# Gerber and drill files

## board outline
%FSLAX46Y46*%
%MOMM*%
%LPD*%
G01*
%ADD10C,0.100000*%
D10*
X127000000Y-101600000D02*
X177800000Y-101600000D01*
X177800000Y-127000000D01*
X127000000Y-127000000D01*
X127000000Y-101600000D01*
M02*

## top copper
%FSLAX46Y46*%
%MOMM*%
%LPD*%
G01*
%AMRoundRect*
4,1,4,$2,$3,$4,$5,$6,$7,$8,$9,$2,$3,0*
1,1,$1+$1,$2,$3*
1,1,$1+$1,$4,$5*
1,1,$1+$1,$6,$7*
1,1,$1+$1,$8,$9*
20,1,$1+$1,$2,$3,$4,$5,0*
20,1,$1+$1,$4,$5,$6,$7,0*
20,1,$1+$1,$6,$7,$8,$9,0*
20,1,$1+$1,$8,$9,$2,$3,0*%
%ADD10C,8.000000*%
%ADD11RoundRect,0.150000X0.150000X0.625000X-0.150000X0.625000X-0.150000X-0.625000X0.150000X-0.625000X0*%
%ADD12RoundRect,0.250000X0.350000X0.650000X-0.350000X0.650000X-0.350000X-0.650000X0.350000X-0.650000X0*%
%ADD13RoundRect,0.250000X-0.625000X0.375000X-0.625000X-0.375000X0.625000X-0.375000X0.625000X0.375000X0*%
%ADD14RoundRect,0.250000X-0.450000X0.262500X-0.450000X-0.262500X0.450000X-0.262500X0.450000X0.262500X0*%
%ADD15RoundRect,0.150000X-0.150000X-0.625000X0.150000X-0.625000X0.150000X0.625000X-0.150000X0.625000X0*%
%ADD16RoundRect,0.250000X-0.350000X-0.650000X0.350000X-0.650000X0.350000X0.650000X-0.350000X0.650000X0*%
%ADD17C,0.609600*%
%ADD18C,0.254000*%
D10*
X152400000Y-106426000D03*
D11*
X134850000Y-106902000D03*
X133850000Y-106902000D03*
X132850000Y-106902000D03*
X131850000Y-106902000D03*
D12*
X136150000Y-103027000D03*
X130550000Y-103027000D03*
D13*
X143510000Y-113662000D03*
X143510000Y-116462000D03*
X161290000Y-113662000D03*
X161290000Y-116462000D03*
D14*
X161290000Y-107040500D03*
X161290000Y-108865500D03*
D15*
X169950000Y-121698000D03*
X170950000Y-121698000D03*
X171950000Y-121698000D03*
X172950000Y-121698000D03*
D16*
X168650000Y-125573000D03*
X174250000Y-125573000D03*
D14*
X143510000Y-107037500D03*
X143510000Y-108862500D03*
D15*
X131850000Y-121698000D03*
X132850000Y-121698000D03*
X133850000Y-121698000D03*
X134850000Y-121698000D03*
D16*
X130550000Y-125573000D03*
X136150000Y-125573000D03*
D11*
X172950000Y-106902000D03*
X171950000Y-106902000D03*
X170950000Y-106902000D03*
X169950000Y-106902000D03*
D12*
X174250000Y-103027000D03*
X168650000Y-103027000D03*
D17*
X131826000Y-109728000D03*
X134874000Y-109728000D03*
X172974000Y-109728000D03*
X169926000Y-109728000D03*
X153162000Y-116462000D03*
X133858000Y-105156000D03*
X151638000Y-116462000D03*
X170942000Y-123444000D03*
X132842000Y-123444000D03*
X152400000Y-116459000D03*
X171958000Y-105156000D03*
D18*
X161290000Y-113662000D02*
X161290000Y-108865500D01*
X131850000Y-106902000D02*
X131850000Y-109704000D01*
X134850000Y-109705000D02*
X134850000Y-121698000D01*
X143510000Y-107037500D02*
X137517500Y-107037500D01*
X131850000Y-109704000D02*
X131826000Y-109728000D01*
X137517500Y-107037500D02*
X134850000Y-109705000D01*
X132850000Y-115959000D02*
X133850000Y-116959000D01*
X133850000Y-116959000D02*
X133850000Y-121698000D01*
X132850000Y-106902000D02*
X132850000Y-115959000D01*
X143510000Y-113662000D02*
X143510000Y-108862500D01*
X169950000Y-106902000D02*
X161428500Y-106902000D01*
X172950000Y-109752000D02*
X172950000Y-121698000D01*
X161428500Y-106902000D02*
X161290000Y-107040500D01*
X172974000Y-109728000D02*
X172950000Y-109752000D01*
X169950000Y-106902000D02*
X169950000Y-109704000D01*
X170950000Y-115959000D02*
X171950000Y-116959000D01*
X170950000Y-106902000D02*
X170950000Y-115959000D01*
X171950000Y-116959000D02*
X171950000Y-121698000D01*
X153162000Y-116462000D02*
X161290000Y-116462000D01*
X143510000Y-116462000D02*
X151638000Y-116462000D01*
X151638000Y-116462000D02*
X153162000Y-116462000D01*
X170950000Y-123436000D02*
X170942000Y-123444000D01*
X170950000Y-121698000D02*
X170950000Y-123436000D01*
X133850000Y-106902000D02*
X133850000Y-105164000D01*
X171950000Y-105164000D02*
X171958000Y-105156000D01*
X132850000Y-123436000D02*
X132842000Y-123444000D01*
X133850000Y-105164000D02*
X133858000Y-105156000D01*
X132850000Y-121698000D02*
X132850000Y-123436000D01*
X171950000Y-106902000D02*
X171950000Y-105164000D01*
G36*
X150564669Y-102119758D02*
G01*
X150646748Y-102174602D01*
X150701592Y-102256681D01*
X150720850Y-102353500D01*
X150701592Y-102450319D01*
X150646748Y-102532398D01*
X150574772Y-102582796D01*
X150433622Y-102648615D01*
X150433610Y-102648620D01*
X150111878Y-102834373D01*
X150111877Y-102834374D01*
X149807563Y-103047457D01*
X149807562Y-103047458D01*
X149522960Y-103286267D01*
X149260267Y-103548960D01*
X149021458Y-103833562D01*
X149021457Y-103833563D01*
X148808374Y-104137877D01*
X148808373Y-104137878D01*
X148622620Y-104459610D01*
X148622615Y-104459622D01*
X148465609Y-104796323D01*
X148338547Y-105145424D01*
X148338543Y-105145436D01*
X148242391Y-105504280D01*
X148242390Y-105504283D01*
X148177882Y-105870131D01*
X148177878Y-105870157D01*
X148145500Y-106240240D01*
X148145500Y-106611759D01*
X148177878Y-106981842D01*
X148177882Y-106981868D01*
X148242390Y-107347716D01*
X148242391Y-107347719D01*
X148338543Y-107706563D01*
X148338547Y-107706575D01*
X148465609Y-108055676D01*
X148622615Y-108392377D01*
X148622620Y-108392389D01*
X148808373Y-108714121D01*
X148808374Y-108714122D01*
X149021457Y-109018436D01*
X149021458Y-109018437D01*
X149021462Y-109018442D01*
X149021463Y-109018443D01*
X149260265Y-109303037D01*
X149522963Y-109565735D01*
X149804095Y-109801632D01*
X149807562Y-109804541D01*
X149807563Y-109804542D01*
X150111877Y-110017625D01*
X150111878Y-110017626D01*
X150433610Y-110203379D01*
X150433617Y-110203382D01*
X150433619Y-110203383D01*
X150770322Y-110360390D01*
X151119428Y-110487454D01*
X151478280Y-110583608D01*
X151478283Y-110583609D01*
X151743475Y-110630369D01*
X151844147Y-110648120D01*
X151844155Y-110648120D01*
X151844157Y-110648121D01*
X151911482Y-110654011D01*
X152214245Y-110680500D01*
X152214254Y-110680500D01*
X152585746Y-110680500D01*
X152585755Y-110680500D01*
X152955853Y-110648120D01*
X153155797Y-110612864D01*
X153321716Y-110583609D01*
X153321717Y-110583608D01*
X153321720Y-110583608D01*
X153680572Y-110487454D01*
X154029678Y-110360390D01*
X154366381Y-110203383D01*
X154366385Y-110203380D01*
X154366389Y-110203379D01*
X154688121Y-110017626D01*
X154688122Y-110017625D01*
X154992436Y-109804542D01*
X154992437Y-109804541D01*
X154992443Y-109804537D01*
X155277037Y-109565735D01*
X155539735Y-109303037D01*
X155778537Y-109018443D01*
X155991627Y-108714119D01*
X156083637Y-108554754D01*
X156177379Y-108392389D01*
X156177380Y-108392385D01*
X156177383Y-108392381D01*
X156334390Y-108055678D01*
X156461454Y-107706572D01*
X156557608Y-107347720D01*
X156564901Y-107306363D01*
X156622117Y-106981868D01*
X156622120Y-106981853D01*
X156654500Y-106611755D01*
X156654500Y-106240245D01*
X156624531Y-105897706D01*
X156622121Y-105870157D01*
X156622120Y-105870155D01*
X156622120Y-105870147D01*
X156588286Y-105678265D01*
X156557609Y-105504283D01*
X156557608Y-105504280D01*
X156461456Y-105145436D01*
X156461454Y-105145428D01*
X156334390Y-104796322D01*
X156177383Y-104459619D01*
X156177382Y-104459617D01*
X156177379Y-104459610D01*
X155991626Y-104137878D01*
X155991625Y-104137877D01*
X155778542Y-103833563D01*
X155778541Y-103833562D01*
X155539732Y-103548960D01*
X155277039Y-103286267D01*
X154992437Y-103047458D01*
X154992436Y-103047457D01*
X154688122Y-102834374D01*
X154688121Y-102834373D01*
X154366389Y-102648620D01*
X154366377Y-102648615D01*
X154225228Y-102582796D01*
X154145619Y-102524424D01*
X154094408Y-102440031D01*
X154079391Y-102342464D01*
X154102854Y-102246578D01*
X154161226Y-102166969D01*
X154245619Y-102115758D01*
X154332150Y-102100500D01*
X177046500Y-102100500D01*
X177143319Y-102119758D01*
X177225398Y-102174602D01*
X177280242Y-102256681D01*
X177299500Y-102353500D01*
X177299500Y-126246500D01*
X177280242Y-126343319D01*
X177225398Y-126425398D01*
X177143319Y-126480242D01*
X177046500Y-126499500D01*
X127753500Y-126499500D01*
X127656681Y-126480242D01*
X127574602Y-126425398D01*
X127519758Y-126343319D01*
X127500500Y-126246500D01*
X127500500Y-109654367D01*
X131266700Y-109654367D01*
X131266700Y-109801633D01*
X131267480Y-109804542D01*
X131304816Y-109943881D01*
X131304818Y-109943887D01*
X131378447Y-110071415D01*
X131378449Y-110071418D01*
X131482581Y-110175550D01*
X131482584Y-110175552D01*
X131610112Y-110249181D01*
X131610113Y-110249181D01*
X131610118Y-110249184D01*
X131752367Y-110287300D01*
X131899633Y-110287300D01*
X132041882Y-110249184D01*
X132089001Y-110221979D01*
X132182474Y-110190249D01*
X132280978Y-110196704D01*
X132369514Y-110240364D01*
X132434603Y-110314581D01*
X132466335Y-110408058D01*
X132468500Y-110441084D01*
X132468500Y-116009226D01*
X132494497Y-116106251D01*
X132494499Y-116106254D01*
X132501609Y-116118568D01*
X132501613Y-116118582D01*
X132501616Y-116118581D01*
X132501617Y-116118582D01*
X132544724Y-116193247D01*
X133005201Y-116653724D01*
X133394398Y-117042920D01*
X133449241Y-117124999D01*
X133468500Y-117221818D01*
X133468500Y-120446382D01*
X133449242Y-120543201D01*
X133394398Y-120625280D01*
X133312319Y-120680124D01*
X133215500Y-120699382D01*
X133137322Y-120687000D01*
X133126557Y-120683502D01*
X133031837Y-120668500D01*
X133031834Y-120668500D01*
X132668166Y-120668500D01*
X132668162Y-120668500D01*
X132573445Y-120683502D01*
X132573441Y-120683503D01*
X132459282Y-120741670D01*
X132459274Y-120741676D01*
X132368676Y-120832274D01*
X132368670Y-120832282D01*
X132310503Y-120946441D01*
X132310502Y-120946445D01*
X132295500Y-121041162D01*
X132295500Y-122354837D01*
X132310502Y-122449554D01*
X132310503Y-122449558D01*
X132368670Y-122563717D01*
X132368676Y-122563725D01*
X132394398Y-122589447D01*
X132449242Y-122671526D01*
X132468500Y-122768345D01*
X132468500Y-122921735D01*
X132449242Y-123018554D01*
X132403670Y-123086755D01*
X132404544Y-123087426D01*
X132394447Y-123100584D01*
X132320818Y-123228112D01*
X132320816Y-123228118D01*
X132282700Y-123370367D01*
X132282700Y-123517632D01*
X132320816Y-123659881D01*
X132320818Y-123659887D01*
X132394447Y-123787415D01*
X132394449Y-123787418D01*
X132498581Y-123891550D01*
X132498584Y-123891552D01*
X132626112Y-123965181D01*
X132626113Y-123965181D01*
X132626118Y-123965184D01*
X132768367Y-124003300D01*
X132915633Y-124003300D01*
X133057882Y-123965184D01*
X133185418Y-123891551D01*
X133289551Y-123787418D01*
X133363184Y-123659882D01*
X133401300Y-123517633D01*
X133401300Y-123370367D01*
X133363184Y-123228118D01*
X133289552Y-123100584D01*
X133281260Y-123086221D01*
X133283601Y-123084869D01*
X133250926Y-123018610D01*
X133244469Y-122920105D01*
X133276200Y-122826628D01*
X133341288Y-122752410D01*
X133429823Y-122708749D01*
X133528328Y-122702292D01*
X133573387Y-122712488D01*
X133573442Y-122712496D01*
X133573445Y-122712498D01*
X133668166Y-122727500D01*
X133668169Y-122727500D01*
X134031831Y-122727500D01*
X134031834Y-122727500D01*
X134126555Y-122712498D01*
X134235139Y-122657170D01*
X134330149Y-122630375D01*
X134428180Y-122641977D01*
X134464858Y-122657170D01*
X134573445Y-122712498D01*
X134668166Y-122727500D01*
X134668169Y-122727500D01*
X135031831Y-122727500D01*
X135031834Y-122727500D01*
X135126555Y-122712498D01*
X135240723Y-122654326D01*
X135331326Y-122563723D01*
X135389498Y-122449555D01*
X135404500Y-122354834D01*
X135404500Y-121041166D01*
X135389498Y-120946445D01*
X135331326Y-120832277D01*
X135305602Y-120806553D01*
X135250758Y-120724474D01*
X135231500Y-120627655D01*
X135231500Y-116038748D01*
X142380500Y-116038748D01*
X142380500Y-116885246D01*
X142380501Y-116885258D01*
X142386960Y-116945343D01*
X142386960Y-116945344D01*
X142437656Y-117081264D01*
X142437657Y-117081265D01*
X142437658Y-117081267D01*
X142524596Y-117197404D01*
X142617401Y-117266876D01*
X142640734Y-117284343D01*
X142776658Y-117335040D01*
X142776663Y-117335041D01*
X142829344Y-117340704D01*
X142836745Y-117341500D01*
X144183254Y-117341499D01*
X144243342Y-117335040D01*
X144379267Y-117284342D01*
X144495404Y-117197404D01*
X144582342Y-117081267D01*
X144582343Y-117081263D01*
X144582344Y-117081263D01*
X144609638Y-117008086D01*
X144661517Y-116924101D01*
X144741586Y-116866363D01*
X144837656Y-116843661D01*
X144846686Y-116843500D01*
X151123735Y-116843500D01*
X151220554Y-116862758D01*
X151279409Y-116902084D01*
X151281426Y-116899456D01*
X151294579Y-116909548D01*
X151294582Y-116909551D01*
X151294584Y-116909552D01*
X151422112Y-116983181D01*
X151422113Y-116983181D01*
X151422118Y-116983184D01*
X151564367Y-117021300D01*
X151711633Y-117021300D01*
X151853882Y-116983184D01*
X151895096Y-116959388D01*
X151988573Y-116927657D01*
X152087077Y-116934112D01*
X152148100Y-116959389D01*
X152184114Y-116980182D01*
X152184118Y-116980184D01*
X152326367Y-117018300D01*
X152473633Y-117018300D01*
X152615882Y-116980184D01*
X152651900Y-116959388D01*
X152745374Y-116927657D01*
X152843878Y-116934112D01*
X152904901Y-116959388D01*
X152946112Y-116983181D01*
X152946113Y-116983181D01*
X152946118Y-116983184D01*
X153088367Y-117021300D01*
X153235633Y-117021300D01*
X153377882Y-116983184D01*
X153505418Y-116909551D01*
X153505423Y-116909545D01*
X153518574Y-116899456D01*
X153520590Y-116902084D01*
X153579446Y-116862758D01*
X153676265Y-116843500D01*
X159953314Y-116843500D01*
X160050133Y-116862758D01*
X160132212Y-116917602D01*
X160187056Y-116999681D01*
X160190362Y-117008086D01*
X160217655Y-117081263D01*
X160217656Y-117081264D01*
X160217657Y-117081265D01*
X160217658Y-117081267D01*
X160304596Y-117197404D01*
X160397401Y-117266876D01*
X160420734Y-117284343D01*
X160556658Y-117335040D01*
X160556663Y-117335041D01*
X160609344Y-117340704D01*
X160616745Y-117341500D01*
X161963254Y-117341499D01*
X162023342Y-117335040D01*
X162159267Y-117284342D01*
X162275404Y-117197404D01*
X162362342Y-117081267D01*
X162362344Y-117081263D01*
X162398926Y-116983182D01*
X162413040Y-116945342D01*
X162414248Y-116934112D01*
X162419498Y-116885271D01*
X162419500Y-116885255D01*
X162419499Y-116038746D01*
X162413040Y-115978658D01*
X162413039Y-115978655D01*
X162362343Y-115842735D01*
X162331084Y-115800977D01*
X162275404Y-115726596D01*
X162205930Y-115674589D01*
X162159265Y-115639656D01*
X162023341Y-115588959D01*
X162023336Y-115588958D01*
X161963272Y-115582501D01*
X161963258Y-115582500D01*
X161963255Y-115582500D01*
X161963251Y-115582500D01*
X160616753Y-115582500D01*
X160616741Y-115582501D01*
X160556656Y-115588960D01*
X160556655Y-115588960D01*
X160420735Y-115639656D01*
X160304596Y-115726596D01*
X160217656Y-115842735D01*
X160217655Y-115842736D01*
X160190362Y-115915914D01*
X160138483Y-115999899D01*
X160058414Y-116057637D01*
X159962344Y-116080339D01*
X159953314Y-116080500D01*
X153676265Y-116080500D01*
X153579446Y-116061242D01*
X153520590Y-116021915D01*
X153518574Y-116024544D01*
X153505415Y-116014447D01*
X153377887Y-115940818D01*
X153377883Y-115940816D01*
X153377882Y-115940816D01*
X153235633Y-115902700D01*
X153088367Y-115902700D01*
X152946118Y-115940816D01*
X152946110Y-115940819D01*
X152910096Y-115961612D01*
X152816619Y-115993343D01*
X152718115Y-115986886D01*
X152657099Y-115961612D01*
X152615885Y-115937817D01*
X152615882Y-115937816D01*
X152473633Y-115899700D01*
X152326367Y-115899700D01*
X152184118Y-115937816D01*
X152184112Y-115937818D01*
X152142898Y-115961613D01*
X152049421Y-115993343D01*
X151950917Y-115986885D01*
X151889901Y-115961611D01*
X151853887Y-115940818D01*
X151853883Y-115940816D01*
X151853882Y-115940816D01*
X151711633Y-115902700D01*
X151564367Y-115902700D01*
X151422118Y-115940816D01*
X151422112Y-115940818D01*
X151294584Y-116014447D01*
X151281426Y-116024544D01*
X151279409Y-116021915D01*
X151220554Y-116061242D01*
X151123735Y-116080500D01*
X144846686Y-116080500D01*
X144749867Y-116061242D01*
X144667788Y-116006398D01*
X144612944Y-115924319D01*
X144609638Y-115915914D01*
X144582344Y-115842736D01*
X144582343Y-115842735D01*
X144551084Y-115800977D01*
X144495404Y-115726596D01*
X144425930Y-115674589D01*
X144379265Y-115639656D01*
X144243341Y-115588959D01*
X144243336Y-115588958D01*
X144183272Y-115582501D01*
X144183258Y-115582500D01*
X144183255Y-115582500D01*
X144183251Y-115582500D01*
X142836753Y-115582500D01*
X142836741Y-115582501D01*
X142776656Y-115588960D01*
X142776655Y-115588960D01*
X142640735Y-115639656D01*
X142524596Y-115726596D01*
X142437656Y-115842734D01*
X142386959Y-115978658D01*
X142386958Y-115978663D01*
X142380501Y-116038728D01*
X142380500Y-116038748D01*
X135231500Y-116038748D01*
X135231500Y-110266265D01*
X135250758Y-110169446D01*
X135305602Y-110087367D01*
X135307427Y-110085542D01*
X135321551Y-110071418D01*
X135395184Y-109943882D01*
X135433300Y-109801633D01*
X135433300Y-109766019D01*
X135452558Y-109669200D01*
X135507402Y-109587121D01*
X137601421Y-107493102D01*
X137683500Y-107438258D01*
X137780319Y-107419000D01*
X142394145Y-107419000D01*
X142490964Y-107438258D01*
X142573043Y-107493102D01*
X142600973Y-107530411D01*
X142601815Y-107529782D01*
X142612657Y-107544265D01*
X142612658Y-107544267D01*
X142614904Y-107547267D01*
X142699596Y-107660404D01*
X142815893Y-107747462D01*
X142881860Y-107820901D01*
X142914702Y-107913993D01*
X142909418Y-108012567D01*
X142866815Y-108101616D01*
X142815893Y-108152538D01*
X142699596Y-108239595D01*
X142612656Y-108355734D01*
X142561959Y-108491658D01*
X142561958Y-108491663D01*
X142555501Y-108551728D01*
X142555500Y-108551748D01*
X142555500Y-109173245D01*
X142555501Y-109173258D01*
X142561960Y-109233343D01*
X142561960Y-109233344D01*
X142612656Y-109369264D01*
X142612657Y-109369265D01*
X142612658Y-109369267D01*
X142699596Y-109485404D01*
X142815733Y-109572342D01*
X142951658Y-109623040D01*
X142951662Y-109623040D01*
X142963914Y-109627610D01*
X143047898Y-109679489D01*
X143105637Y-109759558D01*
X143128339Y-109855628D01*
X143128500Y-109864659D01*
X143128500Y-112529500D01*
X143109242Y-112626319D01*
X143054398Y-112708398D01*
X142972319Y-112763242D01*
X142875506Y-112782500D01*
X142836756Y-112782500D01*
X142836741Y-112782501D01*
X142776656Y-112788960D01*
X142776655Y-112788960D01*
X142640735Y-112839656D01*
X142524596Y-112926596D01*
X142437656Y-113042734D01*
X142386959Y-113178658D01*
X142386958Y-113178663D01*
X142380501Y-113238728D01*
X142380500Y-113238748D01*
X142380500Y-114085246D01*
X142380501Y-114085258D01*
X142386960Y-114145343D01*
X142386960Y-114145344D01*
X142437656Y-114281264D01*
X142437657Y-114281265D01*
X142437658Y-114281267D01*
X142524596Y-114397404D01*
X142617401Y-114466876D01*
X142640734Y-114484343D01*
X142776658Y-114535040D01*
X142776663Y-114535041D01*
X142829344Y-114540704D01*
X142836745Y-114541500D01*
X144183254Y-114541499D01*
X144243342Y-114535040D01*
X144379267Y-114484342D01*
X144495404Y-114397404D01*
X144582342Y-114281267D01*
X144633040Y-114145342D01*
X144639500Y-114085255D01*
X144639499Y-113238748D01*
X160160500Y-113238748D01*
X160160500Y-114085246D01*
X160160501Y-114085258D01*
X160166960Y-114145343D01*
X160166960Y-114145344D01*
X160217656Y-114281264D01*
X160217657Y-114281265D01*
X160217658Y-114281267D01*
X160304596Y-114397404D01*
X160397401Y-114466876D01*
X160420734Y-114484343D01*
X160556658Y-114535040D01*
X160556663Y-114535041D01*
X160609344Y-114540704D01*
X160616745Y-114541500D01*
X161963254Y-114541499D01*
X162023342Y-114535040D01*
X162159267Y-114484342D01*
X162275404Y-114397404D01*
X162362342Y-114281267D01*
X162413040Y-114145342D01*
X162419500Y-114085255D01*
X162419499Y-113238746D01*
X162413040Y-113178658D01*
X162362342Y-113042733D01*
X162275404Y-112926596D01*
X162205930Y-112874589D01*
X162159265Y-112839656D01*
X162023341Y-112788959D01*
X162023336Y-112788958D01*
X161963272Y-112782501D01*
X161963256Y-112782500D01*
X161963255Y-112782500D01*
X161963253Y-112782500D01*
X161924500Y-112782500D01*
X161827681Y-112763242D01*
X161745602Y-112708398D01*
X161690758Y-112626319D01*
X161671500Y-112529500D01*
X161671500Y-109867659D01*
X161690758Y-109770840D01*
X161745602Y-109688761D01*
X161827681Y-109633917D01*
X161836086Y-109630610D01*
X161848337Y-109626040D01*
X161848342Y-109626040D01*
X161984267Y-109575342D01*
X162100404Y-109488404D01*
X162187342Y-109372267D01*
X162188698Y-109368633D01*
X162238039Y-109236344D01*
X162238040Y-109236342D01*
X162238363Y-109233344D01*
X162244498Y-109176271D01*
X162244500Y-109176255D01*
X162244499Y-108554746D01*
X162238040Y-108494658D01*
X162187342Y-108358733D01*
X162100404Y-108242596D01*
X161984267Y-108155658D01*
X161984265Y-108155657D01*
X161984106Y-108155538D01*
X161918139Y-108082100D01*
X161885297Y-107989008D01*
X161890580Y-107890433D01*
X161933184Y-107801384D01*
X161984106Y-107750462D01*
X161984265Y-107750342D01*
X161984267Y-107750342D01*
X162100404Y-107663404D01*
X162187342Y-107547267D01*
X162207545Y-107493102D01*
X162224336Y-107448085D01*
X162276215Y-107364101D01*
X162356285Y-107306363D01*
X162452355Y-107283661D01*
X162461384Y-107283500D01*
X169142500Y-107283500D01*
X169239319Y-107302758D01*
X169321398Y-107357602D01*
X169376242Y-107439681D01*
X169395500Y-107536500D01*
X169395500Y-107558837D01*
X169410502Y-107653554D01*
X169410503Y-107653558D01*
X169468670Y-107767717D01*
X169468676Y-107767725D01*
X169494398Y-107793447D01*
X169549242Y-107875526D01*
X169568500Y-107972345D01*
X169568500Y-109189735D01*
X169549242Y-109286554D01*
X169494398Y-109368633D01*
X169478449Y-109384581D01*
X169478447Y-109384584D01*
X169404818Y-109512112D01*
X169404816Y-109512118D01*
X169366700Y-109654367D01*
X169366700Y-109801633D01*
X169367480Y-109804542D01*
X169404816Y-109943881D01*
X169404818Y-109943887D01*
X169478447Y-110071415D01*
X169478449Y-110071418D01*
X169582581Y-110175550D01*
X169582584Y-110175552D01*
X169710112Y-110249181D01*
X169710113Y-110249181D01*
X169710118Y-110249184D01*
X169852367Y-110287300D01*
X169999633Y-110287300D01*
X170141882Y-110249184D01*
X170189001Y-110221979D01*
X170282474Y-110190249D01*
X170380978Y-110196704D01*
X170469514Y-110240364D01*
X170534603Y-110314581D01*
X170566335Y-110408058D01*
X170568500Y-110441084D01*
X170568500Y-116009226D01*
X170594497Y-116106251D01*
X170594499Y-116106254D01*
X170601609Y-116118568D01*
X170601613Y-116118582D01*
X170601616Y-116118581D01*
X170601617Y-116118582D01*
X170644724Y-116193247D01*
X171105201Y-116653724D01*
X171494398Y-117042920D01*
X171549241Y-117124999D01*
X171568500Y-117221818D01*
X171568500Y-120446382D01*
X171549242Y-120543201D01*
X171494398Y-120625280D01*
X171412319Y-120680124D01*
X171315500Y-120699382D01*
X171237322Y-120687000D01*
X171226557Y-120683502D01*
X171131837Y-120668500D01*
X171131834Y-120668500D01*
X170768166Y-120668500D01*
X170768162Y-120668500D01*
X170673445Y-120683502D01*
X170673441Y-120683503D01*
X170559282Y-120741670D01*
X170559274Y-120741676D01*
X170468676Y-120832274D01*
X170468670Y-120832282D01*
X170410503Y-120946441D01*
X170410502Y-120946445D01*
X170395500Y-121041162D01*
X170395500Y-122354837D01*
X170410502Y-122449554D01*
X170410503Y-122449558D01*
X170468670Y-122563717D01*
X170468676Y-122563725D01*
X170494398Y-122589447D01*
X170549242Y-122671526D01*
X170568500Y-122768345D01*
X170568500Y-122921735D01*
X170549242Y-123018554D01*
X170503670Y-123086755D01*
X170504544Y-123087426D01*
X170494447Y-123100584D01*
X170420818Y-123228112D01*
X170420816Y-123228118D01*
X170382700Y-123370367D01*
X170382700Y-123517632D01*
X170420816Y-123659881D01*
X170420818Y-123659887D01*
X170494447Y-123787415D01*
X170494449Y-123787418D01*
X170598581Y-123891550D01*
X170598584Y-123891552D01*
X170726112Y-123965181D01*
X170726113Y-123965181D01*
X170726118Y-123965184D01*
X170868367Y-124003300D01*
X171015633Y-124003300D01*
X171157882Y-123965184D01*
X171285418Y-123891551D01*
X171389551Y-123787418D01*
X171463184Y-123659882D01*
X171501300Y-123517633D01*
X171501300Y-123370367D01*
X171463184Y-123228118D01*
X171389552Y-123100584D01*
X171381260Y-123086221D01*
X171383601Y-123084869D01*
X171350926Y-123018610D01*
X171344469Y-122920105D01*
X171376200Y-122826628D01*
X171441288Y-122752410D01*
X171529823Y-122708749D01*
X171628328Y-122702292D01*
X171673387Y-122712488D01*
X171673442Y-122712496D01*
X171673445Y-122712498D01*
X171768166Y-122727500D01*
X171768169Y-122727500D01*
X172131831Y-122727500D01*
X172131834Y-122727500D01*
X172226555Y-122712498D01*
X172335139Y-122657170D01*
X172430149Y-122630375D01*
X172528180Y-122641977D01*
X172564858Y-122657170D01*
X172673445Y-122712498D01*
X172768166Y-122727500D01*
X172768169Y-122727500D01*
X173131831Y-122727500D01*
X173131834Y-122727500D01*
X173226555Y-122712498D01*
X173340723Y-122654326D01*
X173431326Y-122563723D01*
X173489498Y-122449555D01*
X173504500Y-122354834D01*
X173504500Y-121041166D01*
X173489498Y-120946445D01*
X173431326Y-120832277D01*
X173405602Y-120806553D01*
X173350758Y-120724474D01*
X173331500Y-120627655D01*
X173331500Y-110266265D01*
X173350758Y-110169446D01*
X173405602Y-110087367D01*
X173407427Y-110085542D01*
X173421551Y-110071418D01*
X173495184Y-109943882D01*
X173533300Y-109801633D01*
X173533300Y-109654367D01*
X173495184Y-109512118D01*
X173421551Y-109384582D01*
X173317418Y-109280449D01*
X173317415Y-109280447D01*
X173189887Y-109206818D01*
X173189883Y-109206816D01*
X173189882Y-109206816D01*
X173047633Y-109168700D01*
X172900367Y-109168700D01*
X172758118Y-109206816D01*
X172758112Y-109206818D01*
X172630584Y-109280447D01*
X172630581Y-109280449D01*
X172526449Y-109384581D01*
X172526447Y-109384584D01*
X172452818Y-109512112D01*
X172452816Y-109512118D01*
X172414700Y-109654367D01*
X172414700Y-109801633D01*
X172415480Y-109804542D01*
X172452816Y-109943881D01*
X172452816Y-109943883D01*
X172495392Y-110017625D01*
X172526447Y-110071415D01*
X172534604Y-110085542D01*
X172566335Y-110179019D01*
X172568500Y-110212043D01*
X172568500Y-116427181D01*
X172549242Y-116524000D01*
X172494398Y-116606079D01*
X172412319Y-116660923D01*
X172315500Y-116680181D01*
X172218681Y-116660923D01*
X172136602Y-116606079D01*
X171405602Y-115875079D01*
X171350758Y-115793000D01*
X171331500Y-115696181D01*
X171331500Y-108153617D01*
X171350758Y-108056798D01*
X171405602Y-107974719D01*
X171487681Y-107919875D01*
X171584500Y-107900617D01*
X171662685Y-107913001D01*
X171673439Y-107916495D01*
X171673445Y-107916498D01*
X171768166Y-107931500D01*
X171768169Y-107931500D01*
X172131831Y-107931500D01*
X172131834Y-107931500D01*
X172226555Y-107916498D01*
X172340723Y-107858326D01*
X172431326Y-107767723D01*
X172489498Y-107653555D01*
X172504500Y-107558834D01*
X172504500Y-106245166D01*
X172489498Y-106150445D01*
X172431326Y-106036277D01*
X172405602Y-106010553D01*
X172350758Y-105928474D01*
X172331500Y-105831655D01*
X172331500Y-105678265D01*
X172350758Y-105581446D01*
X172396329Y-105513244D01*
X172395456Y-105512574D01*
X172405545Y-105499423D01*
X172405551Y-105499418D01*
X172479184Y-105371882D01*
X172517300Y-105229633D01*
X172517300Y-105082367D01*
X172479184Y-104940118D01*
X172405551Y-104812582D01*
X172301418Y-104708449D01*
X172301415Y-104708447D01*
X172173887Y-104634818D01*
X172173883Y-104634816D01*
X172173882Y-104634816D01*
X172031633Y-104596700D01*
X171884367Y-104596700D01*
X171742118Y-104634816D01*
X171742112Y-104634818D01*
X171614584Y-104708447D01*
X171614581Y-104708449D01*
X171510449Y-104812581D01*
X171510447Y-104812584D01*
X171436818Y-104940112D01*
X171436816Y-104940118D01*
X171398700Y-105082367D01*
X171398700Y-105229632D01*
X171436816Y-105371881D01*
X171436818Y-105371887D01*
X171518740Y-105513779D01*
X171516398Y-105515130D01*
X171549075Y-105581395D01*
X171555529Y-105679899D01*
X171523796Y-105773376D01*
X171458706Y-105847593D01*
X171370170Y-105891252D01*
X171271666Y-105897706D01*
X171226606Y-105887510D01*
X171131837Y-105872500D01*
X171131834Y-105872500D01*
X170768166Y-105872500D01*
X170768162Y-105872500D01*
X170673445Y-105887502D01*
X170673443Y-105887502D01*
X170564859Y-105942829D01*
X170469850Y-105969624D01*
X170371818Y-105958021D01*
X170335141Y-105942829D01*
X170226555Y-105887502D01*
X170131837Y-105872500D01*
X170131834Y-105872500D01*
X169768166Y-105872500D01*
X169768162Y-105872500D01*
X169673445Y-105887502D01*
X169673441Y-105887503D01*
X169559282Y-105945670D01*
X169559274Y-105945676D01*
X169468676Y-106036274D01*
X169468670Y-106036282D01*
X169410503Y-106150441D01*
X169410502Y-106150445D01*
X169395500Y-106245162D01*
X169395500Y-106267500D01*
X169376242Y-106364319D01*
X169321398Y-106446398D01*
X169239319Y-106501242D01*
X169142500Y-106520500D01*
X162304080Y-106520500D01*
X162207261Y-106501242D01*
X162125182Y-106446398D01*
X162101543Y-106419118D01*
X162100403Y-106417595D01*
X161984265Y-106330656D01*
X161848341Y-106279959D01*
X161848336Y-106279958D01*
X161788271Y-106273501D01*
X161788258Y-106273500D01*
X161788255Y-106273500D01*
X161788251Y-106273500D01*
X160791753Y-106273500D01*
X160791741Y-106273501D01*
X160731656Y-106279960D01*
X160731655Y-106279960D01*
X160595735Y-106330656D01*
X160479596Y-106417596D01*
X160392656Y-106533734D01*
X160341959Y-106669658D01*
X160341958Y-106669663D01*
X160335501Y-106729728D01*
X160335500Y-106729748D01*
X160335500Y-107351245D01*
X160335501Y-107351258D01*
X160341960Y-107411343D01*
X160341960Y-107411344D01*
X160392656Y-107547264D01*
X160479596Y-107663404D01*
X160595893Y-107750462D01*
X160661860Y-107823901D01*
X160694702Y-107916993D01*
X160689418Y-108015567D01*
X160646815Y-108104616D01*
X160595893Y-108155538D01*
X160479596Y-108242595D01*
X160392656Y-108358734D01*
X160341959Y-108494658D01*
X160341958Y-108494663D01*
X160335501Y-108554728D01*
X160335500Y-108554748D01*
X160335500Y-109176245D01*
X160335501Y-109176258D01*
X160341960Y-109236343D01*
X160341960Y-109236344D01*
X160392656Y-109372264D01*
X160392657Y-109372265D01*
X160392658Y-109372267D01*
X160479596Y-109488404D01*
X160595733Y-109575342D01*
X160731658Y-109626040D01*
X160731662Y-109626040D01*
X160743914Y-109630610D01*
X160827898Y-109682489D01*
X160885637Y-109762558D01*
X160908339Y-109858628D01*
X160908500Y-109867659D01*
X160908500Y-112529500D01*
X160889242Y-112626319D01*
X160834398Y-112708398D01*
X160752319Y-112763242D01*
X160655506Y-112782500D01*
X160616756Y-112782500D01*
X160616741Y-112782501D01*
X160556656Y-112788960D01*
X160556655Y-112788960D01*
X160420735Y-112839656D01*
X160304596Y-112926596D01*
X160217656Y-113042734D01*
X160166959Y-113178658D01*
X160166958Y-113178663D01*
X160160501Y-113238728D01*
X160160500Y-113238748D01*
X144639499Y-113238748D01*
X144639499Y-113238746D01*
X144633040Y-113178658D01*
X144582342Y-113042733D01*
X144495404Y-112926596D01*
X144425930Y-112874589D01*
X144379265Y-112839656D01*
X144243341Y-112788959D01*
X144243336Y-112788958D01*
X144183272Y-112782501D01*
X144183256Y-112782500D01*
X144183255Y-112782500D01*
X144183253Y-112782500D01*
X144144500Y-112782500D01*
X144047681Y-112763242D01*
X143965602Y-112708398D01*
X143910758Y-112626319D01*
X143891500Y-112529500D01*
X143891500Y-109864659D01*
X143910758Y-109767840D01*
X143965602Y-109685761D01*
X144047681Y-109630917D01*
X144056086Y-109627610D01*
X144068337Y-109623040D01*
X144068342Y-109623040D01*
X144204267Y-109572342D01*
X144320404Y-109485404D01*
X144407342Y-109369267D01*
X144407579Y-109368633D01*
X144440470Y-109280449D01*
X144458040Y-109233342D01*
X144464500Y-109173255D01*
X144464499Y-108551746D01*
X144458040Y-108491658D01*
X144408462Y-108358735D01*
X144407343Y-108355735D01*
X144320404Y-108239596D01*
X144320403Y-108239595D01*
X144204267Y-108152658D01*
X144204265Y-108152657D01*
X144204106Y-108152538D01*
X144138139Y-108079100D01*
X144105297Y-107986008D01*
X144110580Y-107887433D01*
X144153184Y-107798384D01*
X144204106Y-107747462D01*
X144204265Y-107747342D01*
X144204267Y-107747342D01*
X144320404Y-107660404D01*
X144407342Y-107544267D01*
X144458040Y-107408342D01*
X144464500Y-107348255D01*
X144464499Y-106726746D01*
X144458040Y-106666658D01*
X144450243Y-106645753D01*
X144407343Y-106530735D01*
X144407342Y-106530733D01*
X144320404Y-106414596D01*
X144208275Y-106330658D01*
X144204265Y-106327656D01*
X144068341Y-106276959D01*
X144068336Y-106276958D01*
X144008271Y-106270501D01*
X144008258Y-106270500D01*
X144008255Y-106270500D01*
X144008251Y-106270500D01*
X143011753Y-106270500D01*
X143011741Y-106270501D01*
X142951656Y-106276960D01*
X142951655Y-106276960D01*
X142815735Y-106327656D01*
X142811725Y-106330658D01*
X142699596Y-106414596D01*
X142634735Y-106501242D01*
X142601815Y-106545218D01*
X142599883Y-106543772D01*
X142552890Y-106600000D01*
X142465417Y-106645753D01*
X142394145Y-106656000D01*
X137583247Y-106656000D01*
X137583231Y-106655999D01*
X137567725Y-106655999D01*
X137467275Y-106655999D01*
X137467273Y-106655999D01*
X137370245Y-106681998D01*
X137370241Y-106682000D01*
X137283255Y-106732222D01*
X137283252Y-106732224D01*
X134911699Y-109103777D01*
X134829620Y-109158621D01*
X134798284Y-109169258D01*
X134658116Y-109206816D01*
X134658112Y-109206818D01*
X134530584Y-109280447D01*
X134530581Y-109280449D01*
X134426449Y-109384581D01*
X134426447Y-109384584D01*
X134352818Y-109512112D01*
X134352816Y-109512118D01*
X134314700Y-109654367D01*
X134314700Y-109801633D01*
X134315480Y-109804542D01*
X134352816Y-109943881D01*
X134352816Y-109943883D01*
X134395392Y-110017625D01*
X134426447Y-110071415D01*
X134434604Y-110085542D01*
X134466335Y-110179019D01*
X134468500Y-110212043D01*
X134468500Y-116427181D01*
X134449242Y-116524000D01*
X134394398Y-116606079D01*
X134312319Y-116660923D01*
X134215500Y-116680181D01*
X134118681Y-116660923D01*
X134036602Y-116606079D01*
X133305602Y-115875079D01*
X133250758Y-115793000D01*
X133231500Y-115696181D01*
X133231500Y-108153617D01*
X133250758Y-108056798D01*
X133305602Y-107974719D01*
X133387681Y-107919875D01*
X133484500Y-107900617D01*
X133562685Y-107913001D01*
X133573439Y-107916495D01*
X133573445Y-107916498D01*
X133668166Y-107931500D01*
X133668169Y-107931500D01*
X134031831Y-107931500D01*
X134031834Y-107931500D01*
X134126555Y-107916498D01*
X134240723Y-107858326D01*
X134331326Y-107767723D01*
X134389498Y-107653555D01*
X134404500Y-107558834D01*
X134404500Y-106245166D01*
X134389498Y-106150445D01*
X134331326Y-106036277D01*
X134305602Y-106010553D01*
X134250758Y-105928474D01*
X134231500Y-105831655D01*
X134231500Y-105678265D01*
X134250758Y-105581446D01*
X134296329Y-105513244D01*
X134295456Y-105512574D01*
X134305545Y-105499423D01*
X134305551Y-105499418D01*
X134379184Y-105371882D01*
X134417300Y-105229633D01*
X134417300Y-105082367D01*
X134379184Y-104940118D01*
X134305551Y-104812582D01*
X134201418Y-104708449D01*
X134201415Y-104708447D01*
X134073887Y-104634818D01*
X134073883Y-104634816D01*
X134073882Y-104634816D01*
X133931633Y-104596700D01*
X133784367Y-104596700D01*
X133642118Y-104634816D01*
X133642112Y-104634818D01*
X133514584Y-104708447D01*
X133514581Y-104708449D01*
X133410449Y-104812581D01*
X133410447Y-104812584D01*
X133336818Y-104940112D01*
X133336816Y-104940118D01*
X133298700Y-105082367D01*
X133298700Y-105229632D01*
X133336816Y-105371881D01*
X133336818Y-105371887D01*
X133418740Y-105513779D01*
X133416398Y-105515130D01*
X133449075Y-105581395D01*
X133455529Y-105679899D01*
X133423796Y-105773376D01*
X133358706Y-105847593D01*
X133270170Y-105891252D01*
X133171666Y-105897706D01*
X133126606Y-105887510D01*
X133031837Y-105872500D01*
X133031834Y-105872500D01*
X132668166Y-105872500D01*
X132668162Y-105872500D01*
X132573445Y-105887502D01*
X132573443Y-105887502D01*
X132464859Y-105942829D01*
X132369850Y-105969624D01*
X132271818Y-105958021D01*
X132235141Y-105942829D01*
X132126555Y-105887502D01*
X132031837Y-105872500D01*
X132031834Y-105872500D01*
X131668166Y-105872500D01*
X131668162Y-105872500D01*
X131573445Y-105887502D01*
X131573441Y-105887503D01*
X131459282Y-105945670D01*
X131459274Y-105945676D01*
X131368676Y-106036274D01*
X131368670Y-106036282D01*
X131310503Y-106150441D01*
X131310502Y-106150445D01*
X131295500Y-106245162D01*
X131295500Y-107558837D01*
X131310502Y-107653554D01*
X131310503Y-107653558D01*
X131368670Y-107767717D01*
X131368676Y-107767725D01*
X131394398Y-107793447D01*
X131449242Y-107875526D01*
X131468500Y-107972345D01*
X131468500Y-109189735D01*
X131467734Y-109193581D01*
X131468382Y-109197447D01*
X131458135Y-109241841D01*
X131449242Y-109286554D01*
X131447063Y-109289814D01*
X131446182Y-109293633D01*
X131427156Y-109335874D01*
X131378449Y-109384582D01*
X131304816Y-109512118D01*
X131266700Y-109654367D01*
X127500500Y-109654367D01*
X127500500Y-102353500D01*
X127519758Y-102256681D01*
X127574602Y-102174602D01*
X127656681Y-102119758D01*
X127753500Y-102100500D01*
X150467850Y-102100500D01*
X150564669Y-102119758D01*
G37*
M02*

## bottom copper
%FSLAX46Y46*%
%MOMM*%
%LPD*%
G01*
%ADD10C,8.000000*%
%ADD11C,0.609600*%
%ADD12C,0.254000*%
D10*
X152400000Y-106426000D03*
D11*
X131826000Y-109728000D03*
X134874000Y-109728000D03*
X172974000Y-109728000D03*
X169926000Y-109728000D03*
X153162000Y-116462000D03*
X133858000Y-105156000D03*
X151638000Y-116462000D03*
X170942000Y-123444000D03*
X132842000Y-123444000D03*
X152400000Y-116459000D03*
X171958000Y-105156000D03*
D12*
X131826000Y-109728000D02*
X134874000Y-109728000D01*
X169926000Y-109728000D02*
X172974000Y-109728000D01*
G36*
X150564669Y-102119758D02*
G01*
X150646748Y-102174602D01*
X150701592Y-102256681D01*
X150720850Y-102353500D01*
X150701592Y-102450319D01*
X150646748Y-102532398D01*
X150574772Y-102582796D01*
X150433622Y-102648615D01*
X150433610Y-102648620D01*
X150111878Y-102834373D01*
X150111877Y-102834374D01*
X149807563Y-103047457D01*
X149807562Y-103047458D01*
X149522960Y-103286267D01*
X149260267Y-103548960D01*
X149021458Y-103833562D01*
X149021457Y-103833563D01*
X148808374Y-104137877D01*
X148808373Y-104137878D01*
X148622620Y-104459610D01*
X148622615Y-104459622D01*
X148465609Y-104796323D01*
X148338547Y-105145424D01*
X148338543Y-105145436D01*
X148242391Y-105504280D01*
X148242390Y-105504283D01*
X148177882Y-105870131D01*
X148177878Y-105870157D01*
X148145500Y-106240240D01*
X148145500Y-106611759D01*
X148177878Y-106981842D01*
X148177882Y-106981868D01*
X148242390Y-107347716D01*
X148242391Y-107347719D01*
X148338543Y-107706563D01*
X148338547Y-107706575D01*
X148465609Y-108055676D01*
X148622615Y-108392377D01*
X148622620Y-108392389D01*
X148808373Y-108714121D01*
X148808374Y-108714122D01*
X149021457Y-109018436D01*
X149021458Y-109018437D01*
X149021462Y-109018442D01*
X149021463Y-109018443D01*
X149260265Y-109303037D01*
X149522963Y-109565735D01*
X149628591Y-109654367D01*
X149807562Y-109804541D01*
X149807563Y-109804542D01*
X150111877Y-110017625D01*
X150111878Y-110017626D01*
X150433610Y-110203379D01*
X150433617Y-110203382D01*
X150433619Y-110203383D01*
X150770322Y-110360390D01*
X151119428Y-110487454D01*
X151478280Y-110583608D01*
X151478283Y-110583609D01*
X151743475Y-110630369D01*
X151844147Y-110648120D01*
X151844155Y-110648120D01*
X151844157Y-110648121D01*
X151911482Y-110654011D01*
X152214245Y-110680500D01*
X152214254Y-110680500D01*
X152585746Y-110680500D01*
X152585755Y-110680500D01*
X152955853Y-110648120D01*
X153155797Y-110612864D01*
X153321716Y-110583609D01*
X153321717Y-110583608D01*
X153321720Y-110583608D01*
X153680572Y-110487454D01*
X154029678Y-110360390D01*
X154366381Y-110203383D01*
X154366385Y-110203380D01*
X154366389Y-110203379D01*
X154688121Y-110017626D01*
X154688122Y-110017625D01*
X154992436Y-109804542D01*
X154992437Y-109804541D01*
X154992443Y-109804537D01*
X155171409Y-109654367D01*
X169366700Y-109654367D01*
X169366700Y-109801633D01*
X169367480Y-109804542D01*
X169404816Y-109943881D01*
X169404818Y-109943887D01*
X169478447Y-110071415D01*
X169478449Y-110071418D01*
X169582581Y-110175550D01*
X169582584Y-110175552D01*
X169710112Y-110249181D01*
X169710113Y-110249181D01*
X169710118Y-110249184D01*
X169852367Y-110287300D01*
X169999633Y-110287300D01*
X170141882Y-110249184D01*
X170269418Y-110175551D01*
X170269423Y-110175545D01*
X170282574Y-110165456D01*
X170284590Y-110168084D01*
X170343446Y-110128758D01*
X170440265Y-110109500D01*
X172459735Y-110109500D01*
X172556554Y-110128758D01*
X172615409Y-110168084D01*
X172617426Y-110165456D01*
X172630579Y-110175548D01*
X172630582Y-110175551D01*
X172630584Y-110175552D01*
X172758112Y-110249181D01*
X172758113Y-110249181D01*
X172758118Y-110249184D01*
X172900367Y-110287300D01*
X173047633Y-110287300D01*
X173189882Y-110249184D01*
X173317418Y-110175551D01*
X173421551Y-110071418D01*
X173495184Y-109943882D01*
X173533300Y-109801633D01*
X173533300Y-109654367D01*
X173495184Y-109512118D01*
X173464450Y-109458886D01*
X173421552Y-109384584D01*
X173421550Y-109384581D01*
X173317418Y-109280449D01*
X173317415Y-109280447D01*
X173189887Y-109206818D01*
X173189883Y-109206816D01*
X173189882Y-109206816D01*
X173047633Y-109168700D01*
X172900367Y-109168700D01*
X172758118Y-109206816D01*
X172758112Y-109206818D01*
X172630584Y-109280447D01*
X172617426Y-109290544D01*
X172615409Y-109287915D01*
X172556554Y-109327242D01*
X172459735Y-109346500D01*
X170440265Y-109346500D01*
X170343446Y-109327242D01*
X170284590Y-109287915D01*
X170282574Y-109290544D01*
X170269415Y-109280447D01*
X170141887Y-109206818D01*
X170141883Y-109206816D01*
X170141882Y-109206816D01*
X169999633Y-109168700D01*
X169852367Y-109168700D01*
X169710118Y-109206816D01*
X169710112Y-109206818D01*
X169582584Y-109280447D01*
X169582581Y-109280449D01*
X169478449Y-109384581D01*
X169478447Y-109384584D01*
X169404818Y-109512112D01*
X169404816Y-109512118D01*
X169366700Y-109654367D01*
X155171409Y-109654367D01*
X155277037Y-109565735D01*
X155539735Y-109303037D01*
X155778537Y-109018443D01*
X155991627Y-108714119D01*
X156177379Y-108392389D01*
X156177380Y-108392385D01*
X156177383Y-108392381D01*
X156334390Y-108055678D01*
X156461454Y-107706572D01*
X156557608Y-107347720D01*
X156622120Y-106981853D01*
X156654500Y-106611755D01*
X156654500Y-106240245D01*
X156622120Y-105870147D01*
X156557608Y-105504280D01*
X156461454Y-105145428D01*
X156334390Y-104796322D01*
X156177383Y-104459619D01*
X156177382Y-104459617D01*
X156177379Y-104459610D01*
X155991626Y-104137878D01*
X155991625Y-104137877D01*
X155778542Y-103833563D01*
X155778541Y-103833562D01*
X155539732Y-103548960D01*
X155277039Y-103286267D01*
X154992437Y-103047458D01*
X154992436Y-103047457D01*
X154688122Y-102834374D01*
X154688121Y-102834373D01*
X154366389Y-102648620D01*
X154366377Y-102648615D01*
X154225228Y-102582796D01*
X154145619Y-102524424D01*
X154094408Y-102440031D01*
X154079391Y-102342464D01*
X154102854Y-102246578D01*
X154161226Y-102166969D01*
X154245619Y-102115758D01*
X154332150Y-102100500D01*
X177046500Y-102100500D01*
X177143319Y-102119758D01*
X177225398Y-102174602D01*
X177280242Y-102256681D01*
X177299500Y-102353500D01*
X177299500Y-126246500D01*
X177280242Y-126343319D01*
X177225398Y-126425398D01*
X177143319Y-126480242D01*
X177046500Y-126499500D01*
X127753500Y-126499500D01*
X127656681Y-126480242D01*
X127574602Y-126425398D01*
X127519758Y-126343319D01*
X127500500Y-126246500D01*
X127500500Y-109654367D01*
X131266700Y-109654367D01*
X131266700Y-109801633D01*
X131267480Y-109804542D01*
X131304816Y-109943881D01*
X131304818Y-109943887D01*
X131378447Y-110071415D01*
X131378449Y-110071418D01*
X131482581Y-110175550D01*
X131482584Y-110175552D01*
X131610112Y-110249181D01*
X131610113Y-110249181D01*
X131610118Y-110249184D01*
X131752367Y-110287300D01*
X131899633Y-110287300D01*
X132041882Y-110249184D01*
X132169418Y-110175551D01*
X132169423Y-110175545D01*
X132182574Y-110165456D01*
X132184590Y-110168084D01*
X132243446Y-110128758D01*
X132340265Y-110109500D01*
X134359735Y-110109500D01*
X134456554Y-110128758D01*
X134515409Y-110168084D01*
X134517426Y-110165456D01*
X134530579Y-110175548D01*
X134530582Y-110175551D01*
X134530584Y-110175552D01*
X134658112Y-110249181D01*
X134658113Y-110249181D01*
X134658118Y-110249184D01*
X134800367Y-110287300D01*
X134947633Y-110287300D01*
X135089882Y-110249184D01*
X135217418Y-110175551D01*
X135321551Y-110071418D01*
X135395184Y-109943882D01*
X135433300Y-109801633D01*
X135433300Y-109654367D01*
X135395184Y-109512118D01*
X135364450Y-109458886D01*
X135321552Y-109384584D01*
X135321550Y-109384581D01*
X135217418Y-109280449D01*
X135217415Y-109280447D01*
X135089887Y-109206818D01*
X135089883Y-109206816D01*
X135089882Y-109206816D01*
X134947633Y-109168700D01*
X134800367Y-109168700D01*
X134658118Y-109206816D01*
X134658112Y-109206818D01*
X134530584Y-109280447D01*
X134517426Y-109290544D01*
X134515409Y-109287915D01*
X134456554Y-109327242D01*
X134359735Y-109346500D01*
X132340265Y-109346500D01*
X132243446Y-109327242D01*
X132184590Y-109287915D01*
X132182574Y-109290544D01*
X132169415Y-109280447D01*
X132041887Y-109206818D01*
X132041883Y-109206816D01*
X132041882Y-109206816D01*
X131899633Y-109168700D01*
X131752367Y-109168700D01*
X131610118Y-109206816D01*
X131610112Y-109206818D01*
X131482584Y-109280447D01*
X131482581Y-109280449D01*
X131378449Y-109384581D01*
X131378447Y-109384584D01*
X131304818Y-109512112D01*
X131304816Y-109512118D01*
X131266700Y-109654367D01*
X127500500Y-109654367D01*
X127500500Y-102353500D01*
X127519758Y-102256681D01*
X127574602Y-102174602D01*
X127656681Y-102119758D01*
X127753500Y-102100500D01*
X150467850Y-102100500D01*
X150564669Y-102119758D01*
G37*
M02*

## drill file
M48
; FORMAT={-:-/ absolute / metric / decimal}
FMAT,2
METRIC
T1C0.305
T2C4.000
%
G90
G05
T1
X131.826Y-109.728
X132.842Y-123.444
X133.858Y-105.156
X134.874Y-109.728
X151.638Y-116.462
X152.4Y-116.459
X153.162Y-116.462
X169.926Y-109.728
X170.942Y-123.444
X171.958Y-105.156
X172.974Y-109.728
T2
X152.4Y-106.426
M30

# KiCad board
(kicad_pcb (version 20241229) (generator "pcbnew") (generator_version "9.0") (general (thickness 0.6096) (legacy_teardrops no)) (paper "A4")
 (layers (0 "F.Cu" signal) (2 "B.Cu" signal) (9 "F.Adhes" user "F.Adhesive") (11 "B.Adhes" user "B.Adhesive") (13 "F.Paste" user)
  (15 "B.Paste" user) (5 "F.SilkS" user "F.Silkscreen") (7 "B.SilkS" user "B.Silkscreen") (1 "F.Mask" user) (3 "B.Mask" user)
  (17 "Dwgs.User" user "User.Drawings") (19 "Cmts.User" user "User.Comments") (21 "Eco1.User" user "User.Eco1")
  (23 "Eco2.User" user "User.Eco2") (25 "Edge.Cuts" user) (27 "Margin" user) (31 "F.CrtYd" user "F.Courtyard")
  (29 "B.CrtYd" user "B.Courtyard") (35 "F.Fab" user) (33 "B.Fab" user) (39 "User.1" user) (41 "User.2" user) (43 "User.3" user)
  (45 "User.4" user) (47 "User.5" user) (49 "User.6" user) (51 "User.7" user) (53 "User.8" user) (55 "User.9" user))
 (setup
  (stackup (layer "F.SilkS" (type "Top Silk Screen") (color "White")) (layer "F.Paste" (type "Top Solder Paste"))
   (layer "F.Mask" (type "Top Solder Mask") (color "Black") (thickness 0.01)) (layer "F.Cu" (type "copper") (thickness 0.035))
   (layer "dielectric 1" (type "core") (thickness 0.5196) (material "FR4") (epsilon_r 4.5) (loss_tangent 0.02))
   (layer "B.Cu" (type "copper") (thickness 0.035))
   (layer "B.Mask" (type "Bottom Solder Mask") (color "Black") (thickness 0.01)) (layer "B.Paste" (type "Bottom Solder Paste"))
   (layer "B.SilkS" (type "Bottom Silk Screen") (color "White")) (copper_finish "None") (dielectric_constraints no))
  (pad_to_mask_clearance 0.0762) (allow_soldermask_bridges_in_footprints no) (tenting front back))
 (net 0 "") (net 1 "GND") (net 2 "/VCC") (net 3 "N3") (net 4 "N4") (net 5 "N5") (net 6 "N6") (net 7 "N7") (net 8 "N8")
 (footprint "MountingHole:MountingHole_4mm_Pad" (layer "F.Cu") (at 152.4 106.426)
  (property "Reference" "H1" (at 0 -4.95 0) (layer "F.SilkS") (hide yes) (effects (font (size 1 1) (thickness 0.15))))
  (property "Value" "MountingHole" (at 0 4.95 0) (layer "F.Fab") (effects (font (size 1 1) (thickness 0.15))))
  (pad "1" thru_hole circle (at 0 0) (size 8 8) (drill 4) (layers "*.Cu" "*.Mask") (remove_unused_layers no) (zone_connect 2)))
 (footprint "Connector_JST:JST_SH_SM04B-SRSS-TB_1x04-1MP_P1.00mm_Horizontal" (layer "F.Cu") (at 133.35 104.902 180)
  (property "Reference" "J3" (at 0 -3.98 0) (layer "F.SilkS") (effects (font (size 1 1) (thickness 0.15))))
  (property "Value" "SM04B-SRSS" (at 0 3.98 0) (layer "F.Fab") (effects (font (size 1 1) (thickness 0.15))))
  (pad "1" smd roundrect (at -1.5 -2 180) (size 0.6 1.55) (layers "F.Cu" "F.Mask" "F.Paste") (roundrect_rratio 0.25) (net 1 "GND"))
  (pad "2" smd roundrect (at -0.5 -2 180) (size 0.6 1.55) (layers "F.Cu" "F.Mask" "F.Paste") (roundrect_rratio 0.25) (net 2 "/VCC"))
  (pad "3" smd roundrect (at 0.5 -2 180) (size 0.6 1.55) (layers "F.Cu" "F.Mask" "F.Paste") (roundrect_rratio 0.25) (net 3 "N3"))
  (pad "4" smd roundrect (at 1.5 -2 180) (size 0.6 1.55) (layers "F.Cu" "F.Mask" "F.Paste") (roundrect_rratio 0.25) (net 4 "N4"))
  (pad "MP" smd roundrect (at -2.8 1.875 180) (size 1.2 1.8) (layers "F.Cu" "F.Mask" "F.Paste") (roundrect_rratio 0.208333) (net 1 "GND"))
  (pad "MP" smd roundrect (at 2.8 1.875 180) (size 1.2 1.8) (layers "F.Cu" "F.Mask" "F.Paste") (roundrect_rratio 0.208333) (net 1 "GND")))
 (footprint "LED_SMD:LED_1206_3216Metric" (layer "F.Cu") (at 143.51 115.062 -90)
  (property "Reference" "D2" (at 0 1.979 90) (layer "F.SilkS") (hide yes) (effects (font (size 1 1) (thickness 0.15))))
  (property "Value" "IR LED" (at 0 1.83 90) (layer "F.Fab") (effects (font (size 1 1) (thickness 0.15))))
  (pad "1" smd roundrect (at -1.4 0 270) (size 1.25 1.75) (layers "F.Cu" "F.Mask" "F.Paste") (roundrect_rratio 0.2) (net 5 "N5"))
  (pad "2" smd roundrect (at 1.4 0 270) (size 1.25 1.75) (layers "F.Cu" "F.Mask" "F.Paste") (roundrect_rratio 0.2) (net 2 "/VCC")))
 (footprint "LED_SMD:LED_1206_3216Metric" (layer "F.Cu") (at 161.29 115.062 -90)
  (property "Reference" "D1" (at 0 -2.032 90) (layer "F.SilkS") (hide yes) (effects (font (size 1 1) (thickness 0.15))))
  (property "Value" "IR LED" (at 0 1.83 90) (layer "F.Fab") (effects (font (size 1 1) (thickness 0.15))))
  (pad "1" smd roundrect (at -1.4 0 270) (size 1.25 1.75) (layers "F.Cu" "F.Mask" "F.Paste") (roundrect_rratio 0.2) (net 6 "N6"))
  (pad "2" smd roundrect (at 1.4 0 270) (size 1.25 1.75) (layers "F.Cu" "F.Mask" "F.Paste") (roundrect_rratio 0.2) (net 2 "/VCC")))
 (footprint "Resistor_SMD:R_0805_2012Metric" (layer "F.Cu") (at 161.29 107.953 -90)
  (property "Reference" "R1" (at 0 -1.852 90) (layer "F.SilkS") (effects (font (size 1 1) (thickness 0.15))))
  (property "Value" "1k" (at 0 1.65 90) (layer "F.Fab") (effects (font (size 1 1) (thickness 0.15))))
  (pad "1" smd roundrect (at -0.9125 0 270) (size 1.025 1.4) (layers "F.Cu" "F.Mask" "F.Paste") (roundrect_rratio 0.243902) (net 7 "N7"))
  (pad "2" smd roundrect (at 0.9125 0 270) (size 1.025 1.4) (layers "F.Cu" "F.Mask" "F.Paste") (roundrect_rratio 0.243902) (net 6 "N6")))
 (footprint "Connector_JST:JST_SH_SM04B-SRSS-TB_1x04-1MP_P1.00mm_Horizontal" (layer "F.Cu") (at 171.45 123.698)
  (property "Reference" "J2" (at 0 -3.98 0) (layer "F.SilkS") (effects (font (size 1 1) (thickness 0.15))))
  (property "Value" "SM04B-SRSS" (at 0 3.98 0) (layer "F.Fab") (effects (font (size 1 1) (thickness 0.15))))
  (pad "1" smd roundrect (at -1.5 -2) (size 0.6 1.55) (layers "F.Cu" "F.Mask" "F.Paste") (roundrect_rratio 0.25) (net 1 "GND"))
  (pad "2" smd roundrect (at -0.5 -2) (size 0.6 1.55) (layers "F.Cu" "F.Mask" "F.Paste") (roundrect_rratio 0.25) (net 2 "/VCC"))
  (pad "3" smd roundrect (at 0.5 -2) (size 0.6 1.55) (layers "F.Cu" "F.Mask" "F.Paste") (roundrect_rratio 0.25) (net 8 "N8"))
  (pad "4" smd roundrect (at 1.5 -2) (size 0.6 1.55) (layers "F.Cu" "F.Mask" "F.Paste") (roundrect_rratio 0.25) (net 7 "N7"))
  (pad "MP" smd roundrect (at -2.8 1.875) (size 1.2 1.8) (layers "F.Cu" "F.Mask" "F.Paste") (roundrect_rratio 0.208333) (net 1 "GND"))
  (pad "MP" smd roundrect (at 2.8 1.875) (size 1.2 1.8) (layers "F.Cu" "F.Mask" "F.Paste") (roundrect_rratio 0.208333) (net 1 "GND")))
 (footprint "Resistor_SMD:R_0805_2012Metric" (layer "F.Cu") (at 143.51 107.95 -90)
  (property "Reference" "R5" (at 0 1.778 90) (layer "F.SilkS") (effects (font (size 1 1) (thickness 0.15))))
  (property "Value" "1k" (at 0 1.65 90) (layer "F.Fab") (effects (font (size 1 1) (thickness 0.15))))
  (pad "1" smd roundrect (at -0.9125 0 270) (size 1.025 1.4) (layers "F.Cu" "F.Mask" "F.Paste") (roundrect_rratio 0.243902) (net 4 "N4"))
  (pad "2" smd roundrect (at 0.9125 0 270) (size 1.025 1.4) (layers "F.Cu" "F.Mask" "F.Paste") (roundrect_rratio 0.243902) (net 5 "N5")))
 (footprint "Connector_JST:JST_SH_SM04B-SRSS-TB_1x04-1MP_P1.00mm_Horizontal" (layer "F.Cu") (at 133.35 123.698)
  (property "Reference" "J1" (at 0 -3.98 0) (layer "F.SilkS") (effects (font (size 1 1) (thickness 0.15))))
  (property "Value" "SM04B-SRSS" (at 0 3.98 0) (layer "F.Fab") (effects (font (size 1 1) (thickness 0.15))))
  (pad "1" smd roundrect (at -1.5 -2) (size 0.6 1.55) (layers "F.Cu" "F.Mask" "F.Paste") (roundrect_rratio 0.25) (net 1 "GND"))
  (pad "2" smd roundrect (at -0.5 -2) (size 0.6 1.55) (layers "F.Cu" "F.Mask" "F.Paste") (roundrect_rratio 0.25) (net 2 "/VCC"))
  (pad "3" smd roundrect (at 0.5 -2) (size 0.6 1.55) (layers "F.Cu" "F.Mask" "F.Paste") (roundrect_rratio 0.25) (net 3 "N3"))
  (pad "4" smd roundrect (at 1.5 -2) (size 0.6 1.55) (layers "F.Cu" "F.Mask" "F.Paste") (roundrect_rratio 0.25) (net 4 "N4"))
  (pad "MP" smd roundrect (at -2.8 1.875) (size 1.2 1.8) (layers "F.Cu" "F.Mask" "F.Paste") (roundrect_rratio 0.208333) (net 1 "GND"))
  (pad "MP" smd roundrect (at 2.8 1.875) (size 1.2 1.8) (layers "F.Cu" "F.Mask" "F.Paste") (roundrect_rratio 0.208333) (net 1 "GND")))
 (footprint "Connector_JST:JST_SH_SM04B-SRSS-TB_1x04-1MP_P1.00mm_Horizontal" (layer "F.Cu") (at 171.45 104.902 180)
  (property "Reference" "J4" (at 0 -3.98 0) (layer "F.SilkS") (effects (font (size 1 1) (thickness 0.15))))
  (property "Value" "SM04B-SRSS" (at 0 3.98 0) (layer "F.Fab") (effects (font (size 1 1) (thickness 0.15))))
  (pad "1" smd roundrect (at -1.5 -2 180) (size 0.6 1.55) (layers "F.Cu" "F.Mask" "F.Paste") (roundrect_rratio 0.25) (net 1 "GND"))
  (pad "2" smd roundrect (at -0.5 -2 180) (size 0.6 1.55) (layers "F.Cu" "F.Mask" "F.Paste") (roundrect_rratio 0.25) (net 2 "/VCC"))
  (pad "3" smd roundrect (at 0.5 -2 180) (size 0.6 1.55) (layers "F.Cu" "F.Mask" "F.Paste") (roundrect_rratio 0.25) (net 8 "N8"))
  (pad "4" smd roundrect (at 1.5 -2 180) (size 0.6 1.55) (layers "F.Cu" "F.Mask" "F.Paste") (roundrect_rratio 0.25) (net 7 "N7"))
  (pad "MP" smd roundrect (at -2.8 1.875 180) (size 1.2 1.8) (layers "F.Cu" "F.Mask" "F.Paste") (roundrect_rratio 0.208333) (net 1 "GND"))
  (pad "MP" smd roundrect (at 2.8 1.875 180) (size 1.2 1.8) (layers "F.Cu" "F.Mask" "F.Paste") (roundrect_rratio 0.208333) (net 1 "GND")))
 (gr_rect (start 127 101.6) (end 177.8 127) (stroke (width 0.1) (type default)) (fill no) (locked yes) (layer "Edge.Cuts"))
 (segment (start 161.29 113.662) (end 161.29 108.8655) (width 0.254) (layer "F.Cu") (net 6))
 (segment (start 131.85 106.902) (end 131.85 109.704) (width 0.254) (layer "F.Cu") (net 4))
 (segment (start 134.85 109.705) (end 134.85 121.698) (width 0.254) (layer "F.Cu") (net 4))
 (segment (start 143.51 107.0375) (end 137.5175 107.0375) (width 0.254) (layer "F.Cu") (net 4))
 (segment (start 131.85 109.704) (end 131.826 109.728) (width 0.254) (layer "F.Cu") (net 4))
 (segment (start 137.5175 107.0375) (end 134.85 109.705) (width 0.254) (layer "F.Cu") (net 4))
 (via (at 131.826 109.728) (size 0.6096) (drill 0.3048) (layers "F.Cu" "B.Cu") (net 4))
 (via (at 134.874 109.728) (size 0.6096) (drill 0.3048) (layers "F.Cu" "B.Cu") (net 4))
 (segment (start 131.826 109.728) (end 134.874 109.728) (width 0.254) (layer "B.Cu") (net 4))
 (segment (start 132.85 115.959) (end 133.85 116.959) (width 0.254) (layer "F.Cu") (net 3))
 (segment (start 133.85 116.959) (end 133.85 121.698) (width 0.254) (layer "F.Cu") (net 3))
 (segment (start 132.85 106.902) (end 132.85 115.959) (width 0.254) (layer "F.Cu") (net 3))
 (segment (start 143.51 113.662) (end 143.51 108.8625) (width 0.254) (layer "F.Cu") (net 5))
 (segment (start 169.95 106.902) (end 161.4285 106.902) (width 0.254) (layer "F.Cu") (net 7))
 (segment (start 172.95 109.752) (end 172.95 121.698) (width 0.254) (layer "F.Cu") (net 7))
 (segment (start 161.4285 106.902) (end 161.29 107.0405) (width 0.254) (layer "F.Cu") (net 7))
 (segment (start 172.974 109.728) (end 172.95 109.752) (width 0.254) (layer "F.Cu") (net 7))
 (segment (start 169.95 106.902) (end 169.95 109.704) (width 0.254) (layer "F.Cu") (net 7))
 (via (at 172.974 109.728) (size 0.6096) (drill 0.3048) (layers "F.Cu" "B.Cu") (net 7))
 (via (at 169.926 109.728) (size 0.6096) (drill 0.3048) (layers "F.Cu" "B.Cu") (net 7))
 (segment (start 169.926 109.728) (end 172.974 109.728) (width 0.254) (layer "B.Cu") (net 7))
 (segment (start 170.95 115.959) (end 171.95 116.959) (width 0.254) (layer "F.Cu") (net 8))
 (segment (start 170.95 106.902) (end 170.95 115.959) (width 0.254) (layer "F.Cu") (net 8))
 (segment (start 171.95 116.959) (end 171.95 121.698) (width 0.254) (layer "F.Cu") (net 8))
 (segment (start 153.162 116.462) (end 161.29 116.462) (width 0.254) (layer "F.Cu") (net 2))
 (segment (start 143.51 116.462) (end 151.638 116.462) (width 0.254) (layer "F.Cu") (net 2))
 (segment (start 151.638 116.462) (end 153.162 116.462) (width 0.254) (layer "F.Cu") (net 2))
 (segment (start 170.95 123.436) (end 170.942 123.444) (width 0.254) (layer "F.Cu") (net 2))
 (segment (start 170.95 121.698) (end 170.95 123.436) (width 0.254) (layer "F.Cu") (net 2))
 (segment (start 133.85 106.902) (end 133.85 105.164) (width 0.254) (layer "F.Cu") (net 2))
 (segment (start 171.95 105.164) (end 171.958 105.156) (width 0.254) (layer "F.Cu") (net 2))
 (segment (start 132.85 123.436) (end 132.842 123.444) (width 0.254) (layer "F.Cu") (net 2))
 (segment (start 133.85 105.164) (end 133.858 105.156) (width 0.254) (layer "F.Cu") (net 2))
 (segment (start 132.85 121.698) (end 132.85 123.436) (width 0.254) (layer "F.Cu") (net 2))
 (segment (start 171.95 106.902) (end 171.95 105.164) (width 0.254) (layer "F.Cu") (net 2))
 (via (at 153.162 116.462) (size 0.6096) (drill 0.3048) (layers "F.Cu" "B.Cu") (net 2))
 (via (at 133.858 105.156) (size 0.6096) (drill 0.3048) (layers "F.Cu" "B.Cu") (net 2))
 (via (at 151.638 116.462) (size 0.6096) (drill 0.3048) (layers "F.Cu" "B.Cu") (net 2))
 (via (at 170.942 123.444) (size 0.6096) (drill 0.3048) (layers "F.Cu" "B.Cu") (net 2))
 (via (at 132.842 123.444) (size 0.6096) (drill 0.3048) (layers "F.Cu" "B.Cu") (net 2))
 (via (at 152.4 116.459) (size 0.6096) (drill 0.3048) (layers "F.Cu" "B.Cu") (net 2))
 (via (at 171.958 105.156) (size 0.6096) (drill 0.3048) (layers "F.Cu" "B.Cu") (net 2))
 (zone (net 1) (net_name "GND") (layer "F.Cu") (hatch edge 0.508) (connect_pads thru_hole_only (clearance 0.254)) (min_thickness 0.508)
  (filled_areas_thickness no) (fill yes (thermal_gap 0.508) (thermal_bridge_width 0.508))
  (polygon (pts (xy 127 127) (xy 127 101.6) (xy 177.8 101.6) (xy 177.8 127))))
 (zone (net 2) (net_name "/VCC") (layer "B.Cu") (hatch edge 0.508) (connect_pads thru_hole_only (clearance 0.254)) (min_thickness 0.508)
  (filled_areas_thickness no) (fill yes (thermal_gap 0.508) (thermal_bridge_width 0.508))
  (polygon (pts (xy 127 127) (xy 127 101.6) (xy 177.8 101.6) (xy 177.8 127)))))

